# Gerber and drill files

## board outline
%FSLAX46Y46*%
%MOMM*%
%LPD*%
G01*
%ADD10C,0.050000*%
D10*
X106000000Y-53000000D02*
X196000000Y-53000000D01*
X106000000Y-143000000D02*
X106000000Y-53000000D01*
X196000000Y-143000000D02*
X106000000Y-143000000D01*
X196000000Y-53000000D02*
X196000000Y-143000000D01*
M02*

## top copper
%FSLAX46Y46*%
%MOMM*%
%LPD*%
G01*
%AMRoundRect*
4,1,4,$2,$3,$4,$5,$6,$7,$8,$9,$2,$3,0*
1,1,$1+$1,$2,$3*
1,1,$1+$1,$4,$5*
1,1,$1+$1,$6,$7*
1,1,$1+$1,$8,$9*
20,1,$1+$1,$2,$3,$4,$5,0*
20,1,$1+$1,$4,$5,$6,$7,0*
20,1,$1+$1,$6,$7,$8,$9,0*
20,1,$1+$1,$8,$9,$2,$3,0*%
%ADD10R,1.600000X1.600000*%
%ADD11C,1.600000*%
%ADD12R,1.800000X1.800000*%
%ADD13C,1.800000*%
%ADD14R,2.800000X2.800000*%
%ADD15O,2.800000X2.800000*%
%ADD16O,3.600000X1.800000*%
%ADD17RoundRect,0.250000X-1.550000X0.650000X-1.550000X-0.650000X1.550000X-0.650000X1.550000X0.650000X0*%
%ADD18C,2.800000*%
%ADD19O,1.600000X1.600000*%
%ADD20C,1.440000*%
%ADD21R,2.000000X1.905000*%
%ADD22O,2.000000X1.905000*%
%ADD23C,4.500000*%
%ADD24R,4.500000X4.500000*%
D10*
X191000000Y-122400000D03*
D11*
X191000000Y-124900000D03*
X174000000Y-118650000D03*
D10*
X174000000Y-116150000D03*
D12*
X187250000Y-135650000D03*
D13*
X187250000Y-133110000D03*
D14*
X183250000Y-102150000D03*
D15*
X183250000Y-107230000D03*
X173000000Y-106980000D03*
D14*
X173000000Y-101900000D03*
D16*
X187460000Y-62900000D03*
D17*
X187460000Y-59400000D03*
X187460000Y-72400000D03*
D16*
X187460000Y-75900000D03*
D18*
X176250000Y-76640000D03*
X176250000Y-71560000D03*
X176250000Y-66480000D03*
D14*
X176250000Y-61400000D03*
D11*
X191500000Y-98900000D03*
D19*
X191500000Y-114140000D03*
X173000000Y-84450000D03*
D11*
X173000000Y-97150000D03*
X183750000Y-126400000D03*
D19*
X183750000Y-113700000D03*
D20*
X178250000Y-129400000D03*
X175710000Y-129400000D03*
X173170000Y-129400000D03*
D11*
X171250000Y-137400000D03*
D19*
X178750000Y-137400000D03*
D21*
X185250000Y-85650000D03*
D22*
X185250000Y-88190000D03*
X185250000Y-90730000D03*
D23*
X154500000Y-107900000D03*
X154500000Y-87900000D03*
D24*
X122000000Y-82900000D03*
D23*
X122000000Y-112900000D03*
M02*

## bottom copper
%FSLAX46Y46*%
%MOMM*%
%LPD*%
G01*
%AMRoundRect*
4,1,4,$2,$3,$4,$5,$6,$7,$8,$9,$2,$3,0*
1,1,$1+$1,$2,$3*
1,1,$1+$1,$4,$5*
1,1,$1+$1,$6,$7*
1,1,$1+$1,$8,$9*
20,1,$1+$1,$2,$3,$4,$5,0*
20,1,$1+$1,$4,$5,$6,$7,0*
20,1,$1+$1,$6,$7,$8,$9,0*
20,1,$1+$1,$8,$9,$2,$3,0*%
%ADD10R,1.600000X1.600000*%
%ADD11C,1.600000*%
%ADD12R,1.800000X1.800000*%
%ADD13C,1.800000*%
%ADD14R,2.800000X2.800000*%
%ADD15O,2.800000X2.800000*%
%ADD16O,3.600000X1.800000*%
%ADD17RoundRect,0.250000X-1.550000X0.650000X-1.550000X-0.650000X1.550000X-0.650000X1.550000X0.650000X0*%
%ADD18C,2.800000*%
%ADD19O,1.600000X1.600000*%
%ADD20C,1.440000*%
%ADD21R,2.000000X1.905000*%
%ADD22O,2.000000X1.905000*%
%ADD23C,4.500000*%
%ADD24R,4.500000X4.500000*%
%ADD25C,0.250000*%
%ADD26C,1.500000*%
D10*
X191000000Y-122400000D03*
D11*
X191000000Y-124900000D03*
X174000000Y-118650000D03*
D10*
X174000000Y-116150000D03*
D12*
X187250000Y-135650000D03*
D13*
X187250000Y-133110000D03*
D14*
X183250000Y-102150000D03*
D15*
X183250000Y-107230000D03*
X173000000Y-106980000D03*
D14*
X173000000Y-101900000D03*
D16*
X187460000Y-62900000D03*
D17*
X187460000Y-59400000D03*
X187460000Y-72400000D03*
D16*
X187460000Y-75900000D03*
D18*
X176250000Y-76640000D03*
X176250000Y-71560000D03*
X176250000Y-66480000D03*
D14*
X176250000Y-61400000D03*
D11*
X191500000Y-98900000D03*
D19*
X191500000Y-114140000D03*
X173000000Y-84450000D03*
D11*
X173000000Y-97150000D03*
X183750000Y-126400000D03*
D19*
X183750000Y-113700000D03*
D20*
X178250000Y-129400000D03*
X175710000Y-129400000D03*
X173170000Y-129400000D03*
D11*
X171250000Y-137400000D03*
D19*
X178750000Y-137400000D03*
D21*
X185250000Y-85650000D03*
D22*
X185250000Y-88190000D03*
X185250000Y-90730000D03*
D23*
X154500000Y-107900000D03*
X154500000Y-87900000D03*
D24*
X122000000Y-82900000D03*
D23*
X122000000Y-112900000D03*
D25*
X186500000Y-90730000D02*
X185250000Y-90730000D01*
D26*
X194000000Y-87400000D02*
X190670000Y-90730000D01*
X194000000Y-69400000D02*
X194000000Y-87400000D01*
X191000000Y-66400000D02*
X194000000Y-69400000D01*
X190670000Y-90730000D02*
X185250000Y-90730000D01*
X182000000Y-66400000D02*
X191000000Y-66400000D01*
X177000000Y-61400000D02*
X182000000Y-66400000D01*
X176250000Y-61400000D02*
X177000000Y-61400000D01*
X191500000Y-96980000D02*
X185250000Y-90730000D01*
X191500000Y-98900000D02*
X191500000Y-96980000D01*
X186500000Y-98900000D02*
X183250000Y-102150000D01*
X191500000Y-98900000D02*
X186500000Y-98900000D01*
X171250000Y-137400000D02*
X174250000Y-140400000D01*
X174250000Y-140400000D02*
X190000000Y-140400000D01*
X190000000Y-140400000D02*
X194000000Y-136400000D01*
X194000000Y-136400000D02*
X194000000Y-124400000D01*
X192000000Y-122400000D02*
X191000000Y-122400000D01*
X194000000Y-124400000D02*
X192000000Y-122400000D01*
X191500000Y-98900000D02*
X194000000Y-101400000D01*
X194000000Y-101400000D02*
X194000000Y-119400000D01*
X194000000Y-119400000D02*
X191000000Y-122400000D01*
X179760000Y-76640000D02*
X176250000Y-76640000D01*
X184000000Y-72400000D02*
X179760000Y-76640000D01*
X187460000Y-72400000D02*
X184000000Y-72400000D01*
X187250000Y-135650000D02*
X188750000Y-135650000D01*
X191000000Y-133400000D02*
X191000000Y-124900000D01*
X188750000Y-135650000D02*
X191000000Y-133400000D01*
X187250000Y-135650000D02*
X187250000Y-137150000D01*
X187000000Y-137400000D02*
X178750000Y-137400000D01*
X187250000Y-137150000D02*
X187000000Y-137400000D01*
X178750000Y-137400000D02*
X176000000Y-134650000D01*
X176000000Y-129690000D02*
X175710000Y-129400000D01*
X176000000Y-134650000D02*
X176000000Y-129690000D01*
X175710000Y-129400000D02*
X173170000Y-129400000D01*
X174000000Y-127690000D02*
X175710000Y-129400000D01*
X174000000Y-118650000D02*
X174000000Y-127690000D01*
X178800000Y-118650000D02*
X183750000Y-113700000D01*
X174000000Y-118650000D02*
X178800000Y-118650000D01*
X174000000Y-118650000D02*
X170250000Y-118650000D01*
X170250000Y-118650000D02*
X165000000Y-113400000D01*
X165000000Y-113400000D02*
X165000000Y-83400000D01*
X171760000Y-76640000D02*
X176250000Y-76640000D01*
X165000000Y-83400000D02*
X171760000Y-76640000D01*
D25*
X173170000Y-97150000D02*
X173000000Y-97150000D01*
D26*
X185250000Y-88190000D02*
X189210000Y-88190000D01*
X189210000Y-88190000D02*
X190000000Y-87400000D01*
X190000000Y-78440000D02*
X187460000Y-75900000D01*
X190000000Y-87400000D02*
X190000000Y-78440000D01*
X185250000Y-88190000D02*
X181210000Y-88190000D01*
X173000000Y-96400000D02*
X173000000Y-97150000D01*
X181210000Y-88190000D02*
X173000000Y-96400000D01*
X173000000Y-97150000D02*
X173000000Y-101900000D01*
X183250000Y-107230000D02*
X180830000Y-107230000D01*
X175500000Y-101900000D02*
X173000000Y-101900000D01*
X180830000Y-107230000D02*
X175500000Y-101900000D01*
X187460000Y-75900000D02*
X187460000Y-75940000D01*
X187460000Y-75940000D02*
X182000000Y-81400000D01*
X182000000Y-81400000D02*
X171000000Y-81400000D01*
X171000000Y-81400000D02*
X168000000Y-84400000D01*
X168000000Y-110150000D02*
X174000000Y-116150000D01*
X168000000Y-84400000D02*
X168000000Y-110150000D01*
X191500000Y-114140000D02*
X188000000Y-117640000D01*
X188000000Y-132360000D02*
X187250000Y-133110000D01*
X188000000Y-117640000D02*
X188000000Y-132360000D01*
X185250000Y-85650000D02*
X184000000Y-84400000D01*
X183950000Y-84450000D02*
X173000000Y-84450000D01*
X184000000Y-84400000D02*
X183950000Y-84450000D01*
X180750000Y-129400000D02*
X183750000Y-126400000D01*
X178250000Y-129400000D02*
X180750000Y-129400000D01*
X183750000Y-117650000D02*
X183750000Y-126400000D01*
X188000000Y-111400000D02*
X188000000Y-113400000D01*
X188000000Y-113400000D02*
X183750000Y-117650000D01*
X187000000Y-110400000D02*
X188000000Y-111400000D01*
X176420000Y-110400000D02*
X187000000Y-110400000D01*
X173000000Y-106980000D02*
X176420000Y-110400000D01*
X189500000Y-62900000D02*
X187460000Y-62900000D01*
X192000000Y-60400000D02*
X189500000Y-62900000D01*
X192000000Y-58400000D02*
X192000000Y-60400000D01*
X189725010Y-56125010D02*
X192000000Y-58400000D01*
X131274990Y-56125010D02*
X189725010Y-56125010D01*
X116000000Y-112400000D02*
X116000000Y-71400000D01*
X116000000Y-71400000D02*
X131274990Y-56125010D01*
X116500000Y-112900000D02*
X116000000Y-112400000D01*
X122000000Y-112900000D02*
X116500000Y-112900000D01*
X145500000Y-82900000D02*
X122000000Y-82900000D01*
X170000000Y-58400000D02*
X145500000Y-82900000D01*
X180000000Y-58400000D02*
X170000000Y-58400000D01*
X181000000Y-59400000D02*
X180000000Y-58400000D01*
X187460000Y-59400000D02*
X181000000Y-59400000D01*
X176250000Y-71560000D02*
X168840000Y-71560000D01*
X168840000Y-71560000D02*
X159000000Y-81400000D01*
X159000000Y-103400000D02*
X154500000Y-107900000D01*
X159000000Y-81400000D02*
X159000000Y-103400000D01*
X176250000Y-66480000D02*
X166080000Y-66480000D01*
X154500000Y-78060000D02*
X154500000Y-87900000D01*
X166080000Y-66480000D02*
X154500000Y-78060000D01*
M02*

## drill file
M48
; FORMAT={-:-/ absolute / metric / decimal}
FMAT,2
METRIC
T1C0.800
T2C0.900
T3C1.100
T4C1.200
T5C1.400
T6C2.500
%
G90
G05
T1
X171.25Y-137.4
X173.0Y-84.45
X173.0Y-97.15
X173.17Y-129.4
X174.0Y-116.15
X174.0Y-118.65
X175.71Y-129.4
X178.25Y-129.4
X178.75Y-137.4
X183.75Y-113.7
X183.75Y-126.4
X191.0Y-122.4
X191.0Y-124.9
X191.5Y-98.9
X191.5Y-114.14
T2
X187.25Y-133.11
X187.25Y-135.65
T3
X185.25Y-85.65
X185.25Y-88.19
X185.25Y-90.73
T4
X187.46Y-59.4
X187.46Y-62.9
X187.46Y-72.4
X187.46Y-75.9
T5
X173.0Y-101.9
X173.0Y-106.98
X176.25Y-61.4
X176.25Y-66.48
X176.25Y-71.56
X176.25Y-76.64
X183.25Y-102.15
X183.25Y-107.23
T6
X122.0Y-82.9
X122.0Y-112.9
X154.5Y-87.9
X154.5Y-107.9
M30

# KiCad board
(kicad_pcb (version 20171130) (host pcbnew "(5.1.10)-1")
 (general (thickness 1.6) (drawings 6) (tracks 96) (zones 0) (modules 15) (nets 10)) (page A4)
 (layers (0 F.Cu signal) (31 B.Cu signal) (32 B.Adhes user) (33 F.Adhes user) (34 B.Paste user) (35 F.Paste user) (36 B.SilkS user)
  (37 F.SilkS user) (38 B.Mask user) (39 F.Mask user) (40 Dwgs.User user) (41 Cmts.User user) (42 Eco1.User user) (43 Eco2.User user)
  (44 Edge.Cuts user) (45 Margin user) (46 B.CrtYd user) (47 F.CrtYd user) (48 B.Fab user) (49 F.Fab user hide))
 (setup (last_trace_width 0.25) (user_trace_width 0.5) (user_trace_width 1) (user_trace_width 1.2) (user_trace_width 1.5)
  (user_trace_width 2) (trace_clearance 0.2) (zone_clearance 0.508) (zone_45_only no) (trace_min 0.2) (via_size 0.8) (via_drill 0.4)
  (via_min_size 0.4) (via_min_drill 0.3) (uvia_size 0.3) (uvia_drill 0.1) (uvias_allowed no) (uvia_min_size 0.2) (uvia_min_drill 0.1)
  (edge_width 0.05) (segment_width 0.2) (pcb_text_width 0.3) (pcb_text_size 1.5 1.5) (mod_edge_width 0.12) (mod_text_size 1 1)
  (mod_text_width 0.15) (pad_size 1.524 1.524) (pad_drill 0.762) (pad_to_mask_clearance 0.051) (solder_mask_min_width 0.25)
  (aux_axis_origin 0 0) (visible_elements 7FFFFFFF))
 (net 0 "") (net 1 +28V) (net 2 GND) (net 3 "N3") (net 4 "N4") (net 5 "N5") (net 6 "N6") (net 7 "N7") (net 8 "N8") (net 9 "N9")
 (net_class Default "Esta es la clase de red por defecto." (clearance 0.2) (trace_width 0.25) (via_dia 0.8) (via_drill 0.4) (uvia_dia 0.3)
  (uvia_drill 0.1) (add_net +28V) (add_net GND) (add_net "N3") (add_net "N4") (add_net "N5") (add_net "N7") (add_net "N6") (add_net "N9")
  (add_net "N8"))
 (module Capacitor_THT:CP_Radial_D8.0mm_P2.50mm (layer F.Cu) (at 191 122.4 270)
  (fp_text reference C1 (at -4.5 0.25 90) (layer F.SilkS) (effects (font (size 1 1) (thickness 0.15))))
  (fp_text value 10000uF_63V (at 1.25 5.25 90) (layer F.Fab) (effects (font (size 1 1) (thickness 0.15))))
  (pad 1 thru_hole rect (at 0 0 270) (size 1.6 1.6) (drill 0.8) (layers *.Cu *.Mask) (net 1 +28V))
  (pad 2 thru_hole circle (at 2.5 0 270) (size 1.6 1.6) (drill 0.8) (layers *.Cu *.Mask) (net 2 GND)))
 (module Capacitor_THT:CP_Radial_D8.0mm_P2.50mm (layer F.Cu) (at 174 116.15 270)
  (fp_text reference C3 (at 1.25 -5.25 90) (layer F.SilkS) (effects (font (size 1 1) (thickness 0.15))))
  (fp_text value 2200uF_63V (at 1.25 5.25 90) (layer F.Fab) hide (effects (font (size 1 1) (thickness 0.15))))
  (pad 2 thru_hole circle (at 2.5 0 270) (size 1.6 1.6) (drill 0.8) (layers *.Cu *.Mask) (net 2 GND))
  (pad 1 thru_hole rect (at 0 0 270) (size 1.6 1.6) (drill 0.8) (layers *.Cu *.Mask) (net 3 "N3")))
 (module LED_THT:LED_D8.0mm (layer F.Cu) (at 187.25 135.65 90)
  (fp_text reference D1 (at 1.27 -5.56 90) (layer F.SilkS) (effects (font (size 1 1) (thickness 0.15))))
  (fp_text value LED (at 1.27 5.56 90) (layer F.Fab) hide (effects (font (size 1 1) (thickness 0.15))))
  (pad 1 thru_hole rect (at 0 0 90) (size 1.8 1.8) (drill 0.9) (layers *.Cu *.Mask) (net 2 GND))
  (pad 2 thru_hole circle (at 2.54 0 90) (size 1.8 1.8) (drill 0.9) (layers *.Cu *.Mask) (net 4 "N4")))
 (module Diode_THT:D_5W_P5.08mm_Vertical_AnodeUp (layer F.Cu) (at 183.25 102.15 270)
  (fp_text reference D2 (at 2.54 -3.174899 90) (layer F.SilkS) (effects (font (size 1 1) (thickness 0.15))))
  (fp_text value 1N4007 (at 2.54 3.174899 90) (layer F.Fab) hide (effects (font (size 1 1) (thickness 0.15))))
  (pad 1 thru_hole rect (at 0 0 270) (size 2.8 2.8) (drill 1.4) (layers *.Cu *.Mask) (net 1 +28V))
  (pad 2 thru_hole oval (at 5.08 0 270) (size 2.8 2.8) (drill 1.4) (layers *.Cu *.Mask) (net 3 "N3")))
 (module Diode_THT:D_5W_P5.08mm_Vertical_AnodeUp (layer F.Cu) (at 173 101.9 270)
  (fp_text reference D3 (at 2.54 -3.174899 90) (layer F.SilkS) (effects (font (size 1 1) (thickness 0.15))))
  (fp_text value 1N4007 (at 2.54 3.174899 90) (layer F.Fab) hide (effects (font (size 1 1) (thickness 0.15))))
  (pad 2 thru_hole oval (at 5.08 0 270) (size 2.8 2.8) (drill 1.4) (layers *.Cu *.Mask) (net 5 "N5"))
  (pad 1 thru_hole rect (at 0 0 270) (size 2.8 2.8) (drill 1.4) (layers *.Cu *.Mask) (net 3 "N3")))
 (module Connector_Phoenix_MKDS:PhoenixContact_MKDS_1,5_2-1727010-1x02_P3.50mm (layer F.Cu) (at 190 59.4 270)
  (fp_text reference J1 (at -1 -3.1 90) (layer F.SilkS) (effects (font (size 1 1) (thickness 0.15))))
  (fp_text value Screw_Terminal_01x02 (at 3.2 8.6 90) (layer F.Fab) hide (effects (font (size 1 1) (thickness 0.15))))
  (pad 2 thru_hole oval (at 3.5 2.54 270) (size 1.8 3.6) (drill 1.2) (layers *.Cu *.Mask) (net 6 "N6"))
  (pad 1 thru_hole roundrect (at 0 2.54 270) (size 1.8 3.6) (drill 1.2) (layers *.Cu *.Mask) (roundrect_rratio 0.1388888888888889)
   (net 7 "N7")))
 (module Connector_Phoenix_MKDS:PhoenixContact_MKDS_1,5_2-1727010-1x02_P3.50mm (layer F.Cu) (at 190 72.4 270)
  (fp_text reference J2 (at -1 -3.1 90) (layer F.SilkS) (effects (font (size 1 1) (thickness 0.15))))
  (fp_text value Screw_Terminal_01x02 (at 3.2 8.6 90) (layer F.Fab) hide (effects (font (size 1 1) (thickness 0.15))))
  (pad 1 thru_hole roundrect (at 0 2.54 270) (size 1.8 3.6) (drill 1.2) (layers *.Cu *.Mask) (roundrect_rratio 0.1388888888888889)
   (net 2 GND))
  (pad 2 thru_hole oval (at 3.5 2.54 270) (size 1.8 3.6) (drill 1.2) (layers *.Cu *.Mask) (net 3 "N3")))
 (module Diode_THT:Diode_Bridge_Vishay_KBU (layer F.Cu) (at 176.25 61.4 270)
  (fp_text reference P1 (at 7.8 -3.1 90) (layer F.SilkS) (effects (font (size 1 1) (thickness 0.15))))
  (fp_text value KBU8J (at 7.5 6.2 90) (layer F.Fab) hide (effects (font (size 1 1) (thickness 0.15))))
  (pad 4 thru_hole circle (at 15.24 0 270) (size 2.8 2.8) (drill 1.4) (layers *.Cu *.Mask) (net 2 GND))
  (pad 3 thru_hole circle (at 10.16 0 270) (size 2.8 2.8) (drill 1.4) (layers *.Cu *.Mask) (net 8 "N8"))
  (pad 2 thru_hole circle (at 5.08 0 270) (size 2.8 2.8) (drill 1.4) (layers *.Cu *.Mask) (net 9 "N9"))
  (pad 1 thru_hole rect (at 0 0 270) (size 2.8 2.8) (drill 1.4) (layers *.Cu *.Mask) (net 1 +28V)))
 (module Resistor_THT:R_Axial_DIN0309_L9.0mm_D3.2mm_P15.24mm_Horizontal (layer F.Cu) (at 191.5 98.9 270)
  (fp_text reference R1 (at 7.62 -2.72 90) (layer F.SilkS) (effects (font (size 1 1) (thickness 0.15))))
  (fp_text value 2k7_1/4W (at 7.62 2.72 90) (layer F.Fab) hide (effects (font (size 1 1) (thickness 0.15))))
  (pad 1 thru_hole circle (at 0 0 270) (size 1.6 1.6) (drill 0.8) (layers *.Cu *.Mask) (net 1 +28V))
  (pad 2 thru_hole oval (at 15.24 0 270) (size 1.6 1.6) (drill 0.8) (layers *.Cu *.Mask) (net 4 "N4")))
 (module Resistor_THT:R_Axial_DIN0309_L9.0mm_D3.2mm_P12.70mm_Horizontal (layer F.Cu) (at 173 97.15 90)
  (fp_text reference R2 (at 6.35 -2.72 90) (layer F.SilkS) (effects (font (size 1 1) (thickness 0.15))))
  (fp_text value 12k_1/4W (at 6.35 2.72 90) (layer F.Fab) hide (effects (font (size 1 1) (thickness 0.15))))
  (pad 2 thru_hole oval (at 12.7 0 90) (size 1.6 1.6) (drill 0.8) (layers *.Cu *.Mask) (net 5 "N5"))
  (pad 1 thru_hole circle (at 0 0 90) (size 1.6 1.6) (drill 0.8) (layers *.Cu *.Mask) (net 3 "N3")))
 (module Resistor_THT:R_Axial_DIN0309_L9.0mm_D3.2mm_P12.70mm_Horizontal (layer F.Cu) (at 183.75 126.4 90)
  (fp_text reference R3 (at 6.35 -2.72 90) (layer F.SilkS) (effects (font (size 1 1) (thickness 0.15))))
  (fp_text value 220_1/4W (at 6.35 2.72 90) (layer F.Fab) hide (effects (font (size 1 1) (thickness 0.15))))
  (pad 1 thru_hole circle (at 0 0 90) (size 1.6 1.6) (drill 0.8) (layers *.Cu *.Mask) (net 5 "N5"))
  (pad 2 thru_hole oval (at 12.7 0 90) (size 1.6 1.6) (drill 0.8) (layers *.Cu *.Mask) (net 2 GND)))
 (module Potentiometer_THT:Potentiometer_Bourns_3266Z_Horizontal (layer F.Cu) (at 178.25 129.4)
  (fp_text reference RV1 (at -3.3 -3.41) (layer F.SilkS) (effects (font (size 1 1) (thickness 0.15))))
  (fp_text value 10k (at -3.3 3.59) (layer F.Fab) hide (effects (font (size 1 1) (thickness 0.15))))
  (pad 1 thru_hole circle (at 0 0) (size 1.44 1.44) (drill 0.8) (layers *.Cu *.Mask) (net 5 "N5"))
  (pad 2 thru_hole circle (at -2.54 0) (size 1.44 1.44) (drill 0.8) (layers *.Cu *.Mask) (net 2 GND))
  (pad 3 thru_hole circle (at -5.08 0) (size 1.44 1.44) (drill 0.8) (layers *.Cu *.Mask) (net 2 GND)))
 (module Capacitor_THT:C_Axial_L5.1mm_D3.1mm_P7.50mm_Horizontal (layer F.Cu) (at 171.25 137.4)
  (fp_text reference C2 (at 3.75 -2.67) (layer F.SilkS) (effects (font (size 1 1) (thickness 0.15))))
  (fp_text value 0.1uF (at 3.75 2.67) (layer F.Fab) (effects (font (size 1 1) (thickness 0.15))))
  (pad 1 thru_hole circle (at 0 0) (size 1.6 1.6) (drill 0.8) (layers *.Cu *.Mask) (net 1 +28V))
  (pad 2 thru_hole oval (at 7.5 0) (size 1.6 1.6) (drill 0.8) (layers *.Cu *.Mask) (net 2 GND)))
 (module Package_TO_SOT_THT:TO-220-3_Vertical (layer F.Cu) (at 185.25 85.65 270)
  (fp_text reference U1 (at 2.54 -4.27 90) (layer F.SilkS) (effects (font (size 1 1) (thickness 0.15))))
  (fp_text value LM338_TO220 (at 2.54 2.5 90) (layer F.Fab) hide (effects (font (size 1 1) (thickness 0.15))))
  (pad 1 thru_hole rect (at 0 0 270) (size 1.905 2) (drill 1.1) (layers *.Cu *.Mask) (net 5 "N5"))
  (pad 2 thru_hole oval (at 2.54 0 270) (size 1.905 2) (drill 1.1) (layers *.Cu *.Mask) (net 3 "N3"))
  (pad 3 thru_hole oval (at 5.08 0 270) (size 1.905 2) (drill 1.1) (layers *.Cu *.Mask) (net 1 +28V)))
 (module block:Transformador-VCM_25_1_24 (layer F.Cu) (at 122 82.9 270)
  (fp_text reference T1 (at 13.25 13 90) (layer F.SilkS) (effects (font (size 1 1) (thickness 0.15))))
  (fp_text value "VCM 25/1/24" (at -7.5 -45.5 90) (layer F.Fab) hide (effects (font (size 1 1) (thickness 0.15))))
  (pad 4 thru_hole circle (at 25 -32.5 270) (size 4.5 4.5) (drill 2.5) (layers *.Cu *.Mask) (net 8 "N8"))
  (pad 3 thru_hole circle (at 5 -32.5 270) (size 4.5 4.5) (drill 2.5) (layers *.Cu *.Mask) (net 9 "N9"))
  (pad 1 thru_hole rect (at 0 0 270) (size 4.5 4.5) (drill 2.5) (layers *.Cu *.Mask) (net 7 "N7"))
  (pad 2 thru_hole circle (at 30 0 270) (size 4.5 4.5) (drill 2.5) (layers *.Cu *.Mask) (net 6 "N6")))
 (gr_line (start 106 53) (end 196 53) (layer Edge.Cuts) (width 0.05))
 (gr_line (start 106 143) (end 106 53) (layer Edge.Cuts) (width 0.05))
 (gr_line (start 196 143) (end 106 143) (layer Edge.Cuts) (width 0.05))
 (gr_line (start 196 53) (end 196 143) (layer Edge.Cuts) (width 0.05))
 (segment (start 186.5 90.73) (end 185.25 90.73) (width 0.25) (layer B.Cu) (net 1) (status 20))
 (segment (start 194 87.4) (end 190.67 90.73) (width 1.5) (layer B.Cu) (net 1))
 (segment (start 194 69.4) (end 194 87.4) (width 1.5) (layer B.Cu) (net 1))
 (segment (start 191 66.4) (end 194 69.4) (width 1.5) (layer B.Cu) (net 1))
 (segment (start 190.67 90.73) (end 185.25 90.73) (width 1.5) (layer B.Cu) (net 1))
 (segment (start 182 66.4) (end 191 66.4) (width 1.5) (layer B.Cu) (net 1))
 (segment (start 177 61.4) (end 182 66.4) (width 1.5) (layer B.Cu) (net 1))
 (segment (start 176.25 61.4) (end 177 61.4) (width 1.5) (layer B.Cu) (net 1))
 (segment (start 191.5 96.98) (end 185.25 90.73) (width 1.5) (layer B.Cu) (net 1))
 (segment (start 191.5 98.9) (end 191.5 96.98) (width 1.5) (layer B.Cu) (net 1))
 (segment (start 186.5 98.9) (end 183.25 102.15) (width 1.5) (layer B.Cu) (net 1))
 (segment (start 191.5 98.9) (end 186.5 98.9) (width 1.5) (layer B.Cu) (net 1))
 (segment (start 171.25 137.4) (end 174.25 140.4) (width 1.5) (layer B.Cu) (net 1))
 (segment (start 174.25 140.4) (end 190 140.4) (width 1.5) (layer B.Cu) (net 1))
 (segment (start 190 140.4) (end 194 136.4) (width 1.5) (layer B.Cu) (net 1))
 (segment (start 194 136.4) (end 194 124.4) (width 1.5) (layer B.Cu) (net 1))
 (segment (start 192 122.4) (end 191 122.4) (width 1.5) (layer B.Cu) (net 1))
 (segment (start 194 124.4) (end 192 122.4) (width 1.5) (layer B.Cu) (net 1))
 (segment (start 191.5 98.9) (end 194 101.4) (width 1.5) (layer B.Cu) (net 1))
 (segment (start 194 101.4) (end 194 119.4) (width 1.5) (layer B.Cu) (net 1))
 (segment (start 194 119.4) (end 191 122.4) (width 1.5) (layer B.Cu) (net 1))
 (segment (start 179.76 76.64) (end 176.25 76.64) (width 1.5) (layer B.Cu) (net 2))
 (segment (start 184 72.4) (end 179.76 76.64) (width 1.5) (layer B.Cu) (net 2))
 (segment (start 187.46 72.4) (end 184 72.4) (width 1.5) (layer B.Cu) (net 2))
 (segment (start 187.25 135.65) (end 188.75 135.65) (width 1.5) (layer B.Cu) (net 2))
 (segment (start 191 133.4) (end 191 124.9) (width 1.5) (layer B.Cu) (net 2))
 (segment (start 188.75 135.65) (end 191 133.4) (width 1.5) (layer B.Cu) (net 2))
 (segment (start 187.25 135.65) (end 187.25 137.15) (width 1.5) (layer B.Cu) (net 2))
 (segment (start 187 137.4) (end 178.75 137.4) (width 1.5) (layer B.Cu) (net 2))
 (segment (start 187.25 137.15) (end 187 137.4) (width 1.5) (layer B.Cu) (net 2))
 (segment (start 178.75 137.4) (end 176 134.65) (width 1.5) (layer B.Cu) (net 2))
 (segment (start 176 129.69) (end 175.71 129.4) (width 1.5) (layer B.Cu) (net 2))
 (segment (start 176 134.65) (end 176 129.69) (width 1.5) (layer B.Cu) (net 2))
 (segment (start 175.71 129.4) (end 173.17 129.4) (width 1.5) (layer B.Cu) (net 2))
 (segment (start 174 127.69) (end 175.71 129.4) (width 1.5) (layer B.Cu) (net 2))
 (segment (start 174 118.65) (end 174 127.69) (width 1.5) (layer B.Cu) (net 2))
 (segment (start 178.8 118.65) (end 183.75 113.7) (width 1.5) (layer B.Cu) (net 2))
 (segment (start 174 118.65) (end 178.8 118.65) (width 1.5) (layer B.Cu) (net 2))
 (segment (start 174 118.65) (end 170.25 118.65) (width 1.5) (layer B.Cu) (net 2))
 (segment (start 170.25 118.65) (end 165 113.4) (width 1.5) (layer B.Cu) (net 2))
 (segment (start 165 113.4) (end 165 83.4) (width 1.5) (layer B.Cu) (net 2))
 (segment (start 171.76 76.64) (end 176.25 76.64) (width 1.5) (layer B.Cu) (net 2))
 (segment (start 165 83.4) (end 171.76 76.64) (width 1.5) (layer B.Cu) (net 2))
 (segment (start 173.17 97.15) (end 173 97.15) (width 0.25) (layer B.Cu) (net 3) (status 30))
 (segment (start 185.25 88.19) (end 189.21 88.19) (width 1.5) (layer B.Cu) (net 3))
 (segment (start 189.21 88.19) (end 190 87.4) (width 1.5) (layer B.Cu) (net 3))
 (segment (start 190 78.44) (end 187.46 75.9) (width 1.5) (layer B.Cu) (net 3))
 (segment (start 190 87.4) (end 190 78.44) (width 1.5) (layer B.Cu) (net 3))
 (segment (start 185.25 88.19) (end 181.21 88.19) (width 1.5) (layer B.Cu) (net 3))
 (segment (start 173 96.4) (end 173 97.15) (width 1.5) (layer B.Cu) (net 3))
 (segment (start 181.21 88.19) (end 173 96.4) (width 1.5) (layer B.Cu) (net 3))
 (segment (start 173 97.15) (end 173 101.9) (width 1.5) (layer B.Cu) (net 3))
 (segment (start 183.25 107.23) (end 180.83 107.23) (width 1.5) (layer B.Cu) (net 3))
 (segment (start 175.5 101.9) (end 173 101.9) (width 1.5) (layer B.Cu) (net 3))
 (segment (start 180.83 107.23) (end 175.5 101.9) (width 1.5) (layer B.Cu) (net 3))
 (segment (start 187.46 75.9) (end 187.46 75.94) (width 1.5) (layer B.Cu) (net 3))
 (segment (start 187.46 75.94) (end 182 81.4) (width 1.5) (layer B.Cu) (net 3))
 (segment (start 182 81.4) (end 171 81.4) (width 1.5) (layer B.Cu) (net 3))
 (segment (start 171 81.4) (end 168 84.4) (width 1.5) (layer B.Cu) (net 3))
 (segment (start 168 110.15) (end 174 116.15) (width 1.5) (layer B.Cu) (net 3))
 (segment (start 168 84.4) (end 168 110.15) (width 1.5) (layer B.Cu) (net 3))
 (segment (start 191.5 114.14) (end 188 117.64) (width 1.5) (layer B.Cu) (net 4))
 (segment (start 188 132.36) (end 187.25 133.11) (width 1.5) (layer B.Cu) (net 4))
 (segment (start 188 117.64) (end 188 132.36) (width 1.5) (layer B.Cu) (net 4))
 (segment (start 185.25 85.65) (end 184 84.4) (width 1.5) (layer B.Cu) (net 5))
 (segment (start 183.95 84.45) (end 173 84.45) (width 1.5) (layer B.Cu) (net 5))
 (segment (start 184 84.4) (end 183.95 84.45) (width 1.5) (layer B.Cu) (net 5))
 (segment (start 180.75 129.4) (end 183.75 126.4) (width 1.5) (layer B.Cu) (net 5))
 (segment (start 178.25 129.4) (end 180.75 129.4) (width 1.5) (layer B.Cu) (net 5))
 (segment (start 183.75 117.65) (end 183.75 126.4) (width 1.5) (layer B.Cu) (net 5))
 (segment (start 188 111.4) (end 188 113.4) (width 1.5) (layer B.Cu) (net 5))
 (segment (start 188 113.4) (end 183.75 117.65) (width 1.5) (layer B.Cu) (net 5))
 (segment (start 187 110.4) (end 188 111.4) (width 1.5) (layer B.Cu) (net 5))
 (segment (start 176.42 110.4) (end 187 110.4) (width 1.5) (layer B.Cu) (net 5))
 (segment (start 173 106.98) (end 176.42 110.4) (width 1.5) (layer B.Cu) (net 5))
 (segment (start 189.5 62.9) (end 187.46 62.9) (width 1.5) (layer B.Cu) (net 6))
 (segment (start 192 60.4) (end 189.5 62.9) (width 1.5) (layer B.Cu) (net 6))
 (segment (start 192 58.4) (end 192 60.4) (width 1.5) (layer B.Cu) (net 6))
 (segment (start 189.72501 56.12501) (end 192 58.4) (width 1.5) (layer B.Cu) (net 6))
 (segment (start 131.27499 56.12501) (end 189.72501 56.12501) (width 1.5) (layer B.Cu) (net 6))
 (segment (start 116 112.4) (end 116 71.4) (width 1.5) (layer B.Cu) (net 6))
 (segment (start 116 71.4) (end 131.27499 56.12501) (width 1.5) (layer B.Cu) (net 6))
 (segment (start 116.5 112.9) (end 116 112.4) (width 1.5) (layer B.Cu) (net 6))
 (segment (start 122 112.9) (end 116.5 112.9) (width 1.5) (layer B.Cu) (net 6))
 (segment (start 145.5 82.9) (end 122 82.9) (width 1.5) (layer B.Cu) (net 7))
 (segment (start 170 58.4) (end 145.5 82.9) (width 1.5) (layer B.Cu) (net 7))
 (segment (start 180 58.4) (end 170 58.4) (width 1.5) (layer B.Cu) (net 7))
 (segment (start 181 59.4) (end 180 58.4) (width 1.5) (layer B.Cu) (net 7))
 (segment (start 187.46 59.4) (end 181 59.4) (width 1.5) (layer B.Cu) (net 7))
 (segment (start 176.25 71.56) (end 168.84 71.56) (width 1.5) (layer B.Cu) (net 8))
 (segment (start 168.84 71.56) (end 159 81.4) (width 1.5) (layer B.Cu) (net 8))
 (segment (start 159 103.4) (end 154.5 107.9) (width 1.5) (layer B.Cu) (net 8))
 (segment (start 159 81.4) (end 159 103.4) (width 1.5) (layer B.Cu) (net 8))
 (segment (start 176.25 66.48) (end 166.08 66.48) (width 1.5) (layer B.Cu) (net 9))
 (segment (start 154.5 78.06) (end 154.5 87.9) (width 1.5) (layer B.Cu) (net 9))
 (segment (start 166.08 66.48) (end 154.5 78.06) (width 1.5) (layer B.Cu) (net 9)))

